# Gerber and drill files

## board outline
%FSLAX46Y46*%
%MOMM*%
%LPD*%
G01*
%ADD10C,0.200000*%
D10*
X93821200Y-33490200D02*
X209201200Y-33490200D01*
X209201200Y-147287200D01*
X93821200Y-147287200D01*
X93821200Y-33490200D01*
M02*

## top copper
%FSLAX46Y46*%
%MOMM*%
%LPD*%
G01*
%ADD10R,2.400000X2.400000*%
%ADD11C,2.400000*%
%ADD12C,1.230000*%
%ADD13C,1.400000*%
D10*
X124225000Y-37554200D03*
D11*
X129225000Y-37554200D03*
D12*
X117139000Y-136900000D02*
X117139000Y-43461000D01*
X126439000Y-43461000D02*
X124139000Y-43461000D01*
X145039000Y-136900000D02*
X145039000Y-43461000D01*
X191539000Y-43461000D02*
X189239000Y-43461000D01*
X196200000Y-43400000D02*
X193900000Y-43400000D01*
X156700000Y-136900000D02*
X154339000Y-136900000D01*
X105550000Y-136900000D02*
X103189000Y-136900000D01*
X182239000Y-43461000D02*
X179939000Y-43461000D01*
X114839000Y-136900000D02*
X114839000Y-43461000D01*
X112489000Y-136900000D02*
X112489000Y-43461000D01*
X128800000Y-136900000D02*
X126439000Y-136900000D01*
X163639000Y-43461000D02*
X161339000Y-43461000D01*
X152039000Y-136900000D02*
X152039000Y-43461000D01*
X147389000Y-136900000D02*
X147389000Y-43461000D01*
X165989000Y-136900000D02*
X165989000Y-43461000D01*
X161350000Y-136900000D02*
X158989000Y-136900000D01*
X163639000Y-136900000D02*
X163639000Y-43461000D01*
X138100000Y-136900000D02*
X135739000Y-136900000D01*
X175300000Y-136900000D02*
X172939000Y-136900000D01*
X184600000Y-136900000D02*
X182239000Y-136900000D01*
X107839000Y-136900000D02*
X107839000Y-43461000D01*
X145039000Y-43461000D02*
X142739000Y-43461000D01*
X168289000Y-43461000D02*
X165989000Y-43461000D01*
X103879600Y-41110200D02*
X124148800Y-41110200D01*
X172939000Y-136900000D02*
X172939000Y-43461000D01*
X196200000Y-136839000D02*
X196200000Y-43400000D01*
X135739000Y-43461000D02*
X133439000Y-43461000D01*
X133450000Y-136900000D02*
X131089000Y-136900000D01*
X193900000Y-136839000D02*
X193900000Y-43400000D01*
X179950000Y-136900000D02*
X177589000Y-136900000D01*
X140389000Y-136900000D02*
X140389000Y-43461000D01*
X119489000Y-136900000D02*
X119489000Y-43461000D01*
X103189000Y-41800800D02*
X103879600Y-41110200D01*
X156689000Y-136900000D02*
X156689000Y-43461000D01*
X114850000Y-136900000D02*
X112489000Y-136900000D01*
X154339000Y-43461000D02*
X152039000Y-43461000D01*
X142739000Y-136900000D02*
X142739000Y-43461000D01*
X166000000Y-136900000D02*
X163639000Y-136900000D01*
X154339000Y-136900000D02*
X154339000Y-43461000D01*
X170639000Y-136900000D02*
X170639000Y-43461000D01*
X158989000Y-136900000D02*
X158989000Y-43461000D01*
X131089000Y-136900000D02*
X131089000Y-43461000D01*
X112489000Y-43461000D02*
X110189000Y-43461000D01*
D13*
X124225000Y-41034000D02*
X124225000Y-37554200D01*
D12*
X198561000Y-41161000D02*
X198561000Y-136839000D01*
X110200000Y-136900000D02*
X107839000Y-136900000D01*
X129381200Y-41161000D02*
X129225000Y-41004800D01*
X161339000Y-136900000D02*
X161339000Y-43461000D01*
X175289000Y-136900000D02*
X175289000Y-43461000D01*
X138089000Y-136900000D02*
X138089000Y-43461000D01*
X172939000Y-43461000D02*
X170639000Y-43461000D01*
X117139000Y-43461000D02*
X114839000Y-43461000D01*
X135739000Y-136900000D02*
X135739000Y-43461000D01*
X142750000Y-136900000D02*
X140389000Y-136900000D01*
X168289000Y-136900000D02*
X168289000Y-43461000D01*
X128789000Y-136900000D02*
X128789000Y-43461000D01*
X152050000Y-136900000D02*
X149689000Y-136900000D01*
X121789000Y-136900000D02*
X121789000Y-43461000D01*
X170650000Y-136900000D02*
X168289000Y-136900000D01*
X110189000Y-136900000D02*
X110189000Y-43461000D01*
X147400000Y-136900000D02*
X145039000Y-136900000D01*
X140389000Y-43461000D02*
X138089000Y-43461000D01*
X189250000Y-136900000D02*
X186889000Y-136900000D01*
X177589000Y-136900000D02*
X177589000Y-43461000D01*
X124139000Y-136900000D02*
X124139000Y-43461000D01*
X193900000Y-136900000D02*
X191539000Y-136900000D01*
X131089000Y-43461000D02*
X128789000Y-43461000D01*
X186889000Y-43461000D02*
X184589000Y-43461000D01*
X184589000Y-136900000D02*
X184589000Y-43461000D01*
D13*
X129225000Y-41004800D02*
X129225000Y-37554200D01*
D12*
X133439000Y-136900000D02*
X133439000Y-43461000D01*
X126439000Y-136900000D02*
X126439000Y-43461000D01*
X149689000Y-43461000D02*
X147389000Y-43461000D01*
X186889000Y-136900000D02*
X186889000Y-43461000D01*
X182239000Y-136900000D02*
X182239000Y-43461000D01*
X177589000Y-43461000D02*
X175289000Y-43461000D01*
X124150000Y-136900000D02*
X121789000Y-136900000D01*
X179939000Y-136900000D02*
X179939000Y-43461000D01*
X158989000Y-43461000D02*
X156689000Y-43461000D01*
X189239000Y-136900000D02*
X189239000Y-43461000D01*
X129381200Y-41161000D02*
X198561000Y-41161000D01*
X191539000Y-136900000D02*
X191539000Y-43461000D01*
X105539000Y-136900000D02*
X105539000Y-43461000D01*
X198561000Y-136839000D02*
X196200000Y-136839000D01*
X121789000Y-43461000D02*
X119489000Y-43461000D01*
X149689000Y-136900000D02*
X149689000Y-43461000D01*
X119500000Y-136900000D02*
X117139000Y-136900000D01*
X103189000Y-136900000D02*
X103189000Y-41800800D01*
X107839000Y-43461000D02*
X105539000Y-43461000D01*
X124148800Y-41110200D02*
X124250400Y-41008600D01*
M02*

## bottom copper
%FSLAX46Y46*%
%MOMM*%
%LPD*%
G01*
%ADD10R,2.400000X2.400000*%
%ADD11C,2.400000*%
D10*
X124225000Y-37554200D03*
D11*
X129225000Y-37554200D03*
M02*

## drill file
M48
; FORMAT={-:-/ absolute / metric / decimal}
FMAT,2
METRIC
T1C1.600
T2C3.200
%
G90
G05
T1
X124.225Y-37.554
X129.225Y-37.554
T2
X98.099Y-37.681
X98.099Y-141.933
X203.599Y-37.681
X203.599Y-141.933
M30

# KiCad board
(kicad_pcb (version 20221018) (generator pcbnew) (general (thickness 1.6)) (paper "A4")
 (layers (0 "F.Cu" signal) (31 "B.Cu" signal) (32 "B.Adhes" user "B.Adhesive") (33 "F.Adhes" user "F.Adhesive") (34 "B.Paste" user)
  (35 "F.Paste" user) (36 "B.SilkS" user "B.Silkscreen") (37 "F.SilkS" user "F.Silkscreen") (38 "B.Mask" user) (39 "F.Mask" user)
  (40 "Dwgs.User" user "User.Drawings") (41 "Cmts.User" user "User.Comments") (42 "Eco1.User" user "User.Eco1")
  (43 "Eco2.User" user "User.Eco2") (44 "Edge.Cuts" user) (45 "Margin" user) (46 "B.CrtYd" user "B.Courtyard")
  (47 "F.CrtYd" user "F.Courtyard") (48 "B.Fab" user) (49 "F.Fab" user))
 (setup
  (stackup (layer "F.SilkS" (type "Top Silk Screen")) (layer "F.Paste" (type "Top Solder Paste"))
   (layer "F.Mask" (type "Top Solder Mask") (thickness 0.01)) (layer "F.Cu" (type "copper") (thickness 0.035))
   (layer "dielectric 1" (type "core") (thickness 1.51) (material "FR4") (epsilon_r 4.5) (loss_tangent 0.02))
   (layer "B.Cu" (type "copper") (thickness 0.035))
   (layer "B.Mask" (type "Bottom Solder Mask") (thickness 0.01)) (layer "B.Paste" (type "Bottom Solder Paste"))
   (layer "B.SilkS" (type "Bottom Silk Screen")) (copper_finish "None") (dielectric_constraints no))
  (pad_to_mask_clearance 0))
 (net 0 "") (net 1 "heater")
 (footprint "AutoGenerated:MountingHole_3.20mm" (layer "F.Cu") (at 178.0992 89.9332)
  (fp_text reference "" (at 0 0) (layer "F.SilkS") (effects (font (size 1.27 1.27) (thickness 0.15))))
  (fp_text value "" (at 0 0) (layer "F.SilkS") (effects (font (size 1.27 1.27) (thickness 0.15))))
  (pad "" np_thru_hole circle (at 25.5 52) (size 3.2 3.2) (drill 3.2) (layers "F&B.Cu" "*.Mask")))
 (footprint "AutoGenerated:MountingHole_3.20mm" (layer "F.Cu") (at 98.0992 37.6812)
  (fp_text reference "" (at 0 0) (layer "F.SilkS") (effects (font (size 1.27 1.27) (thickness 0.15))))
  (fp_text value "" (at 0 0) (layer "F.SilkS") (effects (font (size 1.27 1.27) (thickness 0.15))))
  (pad "" np_thru_hole circle (at 0 0) (size 3.2 3.2) (drill 3.2) (layers "*.Cu" "*.Mask")))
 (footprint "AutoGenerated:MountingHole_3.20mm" (layer "F.Cu") (at 178.0992 37.6812)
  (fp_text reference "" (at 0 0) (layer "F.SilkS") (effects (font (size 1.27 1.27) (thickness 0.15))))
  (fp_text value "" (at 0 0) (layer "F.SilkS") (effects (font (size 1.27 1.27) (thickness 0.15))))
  (pad "" np_thru_hole circle (at 25.5 0) (size 3.2 3.2) (drill 3.2) (layers "F&B.Cu" "*.Mask")))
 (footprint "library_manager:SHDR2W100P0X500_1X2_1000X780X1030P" (layer "F.Cu") (at 124.225 37.5542)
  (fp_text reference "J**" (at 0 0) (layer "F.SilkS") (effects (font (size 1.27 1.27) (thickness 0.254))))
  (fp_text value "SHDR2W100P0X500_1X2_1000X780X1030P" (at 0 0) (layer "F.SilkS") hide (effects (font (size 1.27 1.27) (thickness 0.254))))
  (pad "1" thru_hole rect (at 0 0) (size 2.4 2.4) (drill 1.6) (layers "*.Cu" "*.Mask") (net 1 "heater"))
  (pad "2" thru_hole circle (at 5 0) (size 2.4 2.4) (drill 1.6) (layers "*.Cu" "*.Mask") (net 1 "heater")))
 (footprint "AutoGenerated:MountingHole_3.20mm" (layer "F.Cu") (at 98.0992 89.9332)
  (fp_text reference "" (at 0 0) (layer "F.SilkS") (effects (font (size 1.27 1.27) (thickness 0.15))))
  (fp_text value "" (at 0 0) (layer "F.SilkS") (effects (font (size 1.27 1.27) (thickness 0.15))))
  (pad "" np_thru_hole circle (at 0 52) (size 3.2 3.2) (drill 3.2) (layers "F&B.Cu" "*.Mask")))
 (gr_rect (start 93.8212 33.4902) (end 209.2012 147.2872) (stroke (width 0.2) (type solid)) (fill none) (layer "Edge.Cuts"))
 (segment (start 117.139 136.9) (end 117.139 43.461) (width 1.23) (layer "F.Cu") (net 1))
 (segment (start 126.439 43.461) (end 124.139 43.461) (width 1.23) (layer "F.Cu") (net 1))
 (segment (start 145.039 136.9) (end 145.039 43.461) (width 1.23) (layer "F.Cu") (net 1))
 (segment (start 191.539 43.461) (end 189.239 43.461) (width 1.23) (layer "F.Cu") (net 1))
 (segment (start 196.2 43.4) (end 193.9 43.4) (width 1.23) (layer "F.Cu") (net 1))
 (segment (start 156.7 136.9) (end 154.339 136.9) (width 1.23) (layer "F.Cu") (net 1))
 (segment (start 105.55 136.9) (end 103.189 136.9) (width 1.23) (layer "F.Cu") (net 1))
 (segment (start 182.239 43.461) (end 179.939 43.461) (width 1.23) (layer "F.Cu") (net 1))
 (segment (start 114.839 136.9) (end 114.839 43.461) (width 1.23) (layer "F.Cu") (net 1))
 (segment (start 112.489 136.9) (end 112.489 43.461) (width 1.23) (layer "F.Cu") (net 1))
 (segment (start 128.8 136.9) (end 126.439 136.9) (width 1.23) (layer "F.Cu") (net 1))
 (segment (start 163.639 43.461) (end 161.339 43.461) (width 1.23) (layer "F.Cu") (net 1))
 (segment (start 152.039 136.9) (end 152.039 43.461) (width 1.23) (layer "F.Cu") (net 1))
 (segment (start 147.389 136.9) (end 147.389 43.461) (width 1.23) (layer "F.Cu") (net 1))
 (segment (start 165.989 136.9) (end 165.989 43.461) (width 1.23) (layer "F.Cu") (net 1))
 (segment (start 161.35 136.9) (end 158.989 136.9) (width 1.23) (layer "F.Cu") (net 1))
 (segment (start 163.639 136.9) (end 163.639 43.461) (width 1.23) (layer "F.Cu") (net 1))
 (segment (start 138.1 136.9) (end 135.739 136.9) (width 1.23) (layer "F.Cu") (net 1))
 (segment (start 175.3 136.9) (end 172.939 136.9) (width 1.23) (layer "F.Cu") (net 1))
 (segment (start 184.6 136.9) (end 182.239 136.9) (width 1.23) (layer "F.Cu") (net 1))
 (segment (start 107.839 136.9) (end 107.839 43.461) (width 1.23) (layer "F.Cu") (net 1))
 (segment (start 145.039 43.461) (end 142.739 43.461) (width 1.23) (layer "F.Cu") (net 1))
 (segment (start 168.289 43.461) (end 165.989 43.461) (width 1.23) (layer "F.Cu") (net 1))
 (segment (start 103.8796 41.1102) (end 124.1488 41.1102) (width 1.23) (layer "F.Cu") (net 1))
 (segment (start 172.939 136.9) (end 172.939 43.461) (width 1.23) (layer "F.Cu") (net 1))
 (segment (start 196.2 136.839) (end 196.2 43.4) (width 1.23) (layer "F.Cu") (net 1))
 (segment (start 135.739 43.461) (end 133.439 43.461) (width 1.23) (layer "F.Cu") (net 1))
 (segment (start 133.45 136.9) (end 131.089 136.9) (width 1.23) (layer "F.Cu") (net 1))
 (segment (start 193.9 136.839) (end 193.9 43.4) (width 1.23) (layer "F.Cu") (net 1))
 (segment (start 179.95 136.9) (end 177.589 136.9) (width 1.23) (layer "F.Cu") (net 1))
 (segment (start 140.389 136.9) (end 140.389 43.461) (width 1.23) (layer "F.Cu") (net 1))
 (segment (start 119.489 136.9) (end 119.489 43.461) (width 1.23) (layer "F.Cu") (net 1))
 (segment (start 103.189 41.8008) (end 103.8796 41.1102) (width 1.23) (layer "F.Cu") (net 1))
 (segment (start 156.689 136.9) (end 156.689 43.461) (width 1.23) (layer "F.Cu") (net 1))
 (segment (start 114.85 136.9) (end 112.489 136.9) (width 1.23) (layer "F.Cu") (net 1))
 (segment (start 154.339 43.461) (end 152.039 43.461) (width 1.23) (layer "F.Cu") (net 1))
 (segment (start 142.739 136.9) (end 142.739 43.461) (width 1.23) (layer "F.Cu") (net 1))
 (segment (start 166 136.9) (end 163.639 136.9) (width 1.23) (layer "F.Cu") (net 1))
 (segment (start 154.339 136.9) (end 154.339 43.461) (width 1.23) (layer "F.Cu") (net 1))
 (segment (start 170.639 136.9) (end 170.639 43.461) (width 1.23) (layer "F.Cu") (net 1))
 (segment (start 158.989 136.9) (end 158.989 43.461) (width 1.23) (layer "F.Cu") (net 1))
 (segment (start 131.089 136.9) (end 131.089 43.461) (width 1.23) (layer "F.Cu") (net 1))
 (segment (start 112.489 43.461) (end 110.189 43.461) (width 1.23) (layer "F.Cu") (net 1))
 (segment (start 124.225 41.034) (end 124.225 37.5542) (width 1.4) (layer "F.Cu") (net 1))
 (segment (start 198.561 41.161) (end 198.561 136.839) (width 1.23) (layer "F.Cu") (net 1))
 (segment (start 110.2 136.9) (end 107.839 136.9) (width 1.23) (layer "F.Cu") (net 1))
 (segment (start 129.3812 41.161) (end 129.225 41.0048) (width 1.23) (layer "F.Cu") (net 1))
 (segment (start 161.339 136.9) (end 161.339 43.461) (width 1.23) (layer "F.Cu") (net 1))
 (segment (start 175.289 136.9) (end 175.289 43.461) (width 1.23) (layer "F.Cu") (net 1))
 (segment (start 138.089 136.9) (end 138.089 43.461) (width 1.23) (layer "F.Cu") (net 1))
 (segment (start 172.939 43.461) (end 170.639 43.461) (width 1.23) (layer "F.Cu") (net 1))
 (segment (start 117.139 43.461) (end 114.839 43.461) (width 1.23) (layer "F.Cu") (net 1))
 (segment (start 135.739 136.9) (end 135.739 43.461) (width 1.23) (layer "F.Cu") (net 1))
 (segment (start 142.75 136.9) (end 140.389 136.9) (width 1.23) (layer "F.Cu") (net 1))
 (segment (start 168.289 136.9) (end 168.289 43.461) (width 1.23) (layer "F.Cu") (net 1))
 (segment (start 128.789 136.9) (end 128.789 43.461) (width 1.23) (layer "F.Cu") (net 1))
 (segment (start 152.05 136.9) (end 149.689 136.9) (width 1.23) (layer "F.Cu") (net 1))
 (segment (start 121.789 136.9) (end 121.789 43.461) (width 1.23) (layer "F.Cu") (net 1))
 (segment (start 170.65 136.9) (end 168.289 136.9) (width 1.23) (layer "F.Cu") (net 1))
 (segment (start 110.189 136.9) (end 110.189 43.461) (width 1.23) (layer "F.Cu") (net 1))
 (segment (start 147.4 136.9) (end 145.039 136.9) (width 1.23) (layer "F.Cu") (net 1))
 (segment (start 140.389 43.461) (end 138.089 43.461) (width 1.23) (layer "F.Cu") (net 1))
 (segment (start 189.25 136.9) (end 186.889 136.9) (width 1.23) (layer "F.Cu") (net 1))
 (segment (start 177.589 136.9) (end 177.589 43.461) (width 1.23) (layer "F.Cu") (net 1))
 (segment (start 124.139 136.9) (end 124.139 43.461) (width 1.23) (layer "F.Cu") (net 1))
 (segment (start 193.9 136.9) (end 191.539 136.9) (width 1.23) (layer "F.Cu") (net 1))
 (segment (start 131.089 43.461) (end 128.789 43.461) (width 1.23) (layer "F.Cu") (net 1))
 (segment (start 186.889 43.461) (end 184.589 43.461) (width 1.23) (layer "F.Cu") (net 1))
 (segment (start 184.589 136.9) (end 184.589 43.461) (width 1.23) (layer "F.Cu") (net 1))
 (segment (start 129.225 41.0048) (end 129.225 37.5542) (width 1.4) (layer "F.Cu") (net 1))
 (segment (start 133.439 136.9) (end 133.439 43.461) (width 1.23) (layer "F.Cu") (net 1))
 (segment (start 126.439 136.9) (end 126.439 43.461) (width 1.23) (layer "F.Cu") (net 1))
 (segment (start 149.689 43.461) (end 147.389 43.461) (width 1.23) (layer "F.Cu") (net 1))
 (segment (start 186.889 136.9) (end 186.889 43.461) (width 1.23) (layer "F.Cu") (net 1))
 (segment (start 182.239 136.9) (end 182.239 43.461) (width 1.23) (layer "F.Cu") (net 1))
 (segment (start 177.589 43.461) (end 175.289 43.461) (width 1.23) (layer "F.Cu") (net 1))
 (segment (start 124.15 136.9) (end 121.789 136.9) (width 1.23) (layer "F.Cu") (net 1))
 (segment (start 179.939 136.9) (end 179.939 43.461) (width 1.23) (layer "F.Cu") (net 1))
 (segment (start 158.989 43.461) (end 156.689 43.461) (width 1.23) (layer "F.Cu") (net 1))
 (segment (start 189.239 136.9) (end 189.239 43.461) (width 1.23) (layer "F.Cu") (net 1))
 (segment (start 129.3812 41.161) (end 198.561 41.161) (width 1.23) (layer "F.Cu") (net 1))
 (segment (start 191.539 136.9) (end 191.539 43.461) (width 1.23) (layer "F.Cu") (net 1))
 (segment (start 105.539 136.9) (end 105.539 43.461) (width 1.23) (layer "F.Cu") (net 1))
 (segment (start 198.561 136.839) (end 196.2 136.839) (width 1.23) (layer "F.Cu") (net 1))
 (segment (start 121.789 43.461) (end 119.489 43.461) (width 1.23) (layer "F.Cu") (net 1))
 (segment (start 149.689 136.9) (end 149.689 43.461) (width 1.23) (layer "F.Cu") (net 1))
 (segment (start 119.5 136.9) (end 117.139 136.9) (width 1.23) (layer "F.Cu") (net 1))
 (segment (start 103.189 136.9) (end 103.189 41.8008) (width 1.23) (layer "F.Cu") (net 1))
 (segment (start 107.839 43.461) (end 105.539 43.461) (width 1.23) (layer "F.Cu") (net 1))
 (segment (start 124.1488 41.1102) (end 124.2504 41.0086) (width 1.23) (layer "F.Cu") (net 1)))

